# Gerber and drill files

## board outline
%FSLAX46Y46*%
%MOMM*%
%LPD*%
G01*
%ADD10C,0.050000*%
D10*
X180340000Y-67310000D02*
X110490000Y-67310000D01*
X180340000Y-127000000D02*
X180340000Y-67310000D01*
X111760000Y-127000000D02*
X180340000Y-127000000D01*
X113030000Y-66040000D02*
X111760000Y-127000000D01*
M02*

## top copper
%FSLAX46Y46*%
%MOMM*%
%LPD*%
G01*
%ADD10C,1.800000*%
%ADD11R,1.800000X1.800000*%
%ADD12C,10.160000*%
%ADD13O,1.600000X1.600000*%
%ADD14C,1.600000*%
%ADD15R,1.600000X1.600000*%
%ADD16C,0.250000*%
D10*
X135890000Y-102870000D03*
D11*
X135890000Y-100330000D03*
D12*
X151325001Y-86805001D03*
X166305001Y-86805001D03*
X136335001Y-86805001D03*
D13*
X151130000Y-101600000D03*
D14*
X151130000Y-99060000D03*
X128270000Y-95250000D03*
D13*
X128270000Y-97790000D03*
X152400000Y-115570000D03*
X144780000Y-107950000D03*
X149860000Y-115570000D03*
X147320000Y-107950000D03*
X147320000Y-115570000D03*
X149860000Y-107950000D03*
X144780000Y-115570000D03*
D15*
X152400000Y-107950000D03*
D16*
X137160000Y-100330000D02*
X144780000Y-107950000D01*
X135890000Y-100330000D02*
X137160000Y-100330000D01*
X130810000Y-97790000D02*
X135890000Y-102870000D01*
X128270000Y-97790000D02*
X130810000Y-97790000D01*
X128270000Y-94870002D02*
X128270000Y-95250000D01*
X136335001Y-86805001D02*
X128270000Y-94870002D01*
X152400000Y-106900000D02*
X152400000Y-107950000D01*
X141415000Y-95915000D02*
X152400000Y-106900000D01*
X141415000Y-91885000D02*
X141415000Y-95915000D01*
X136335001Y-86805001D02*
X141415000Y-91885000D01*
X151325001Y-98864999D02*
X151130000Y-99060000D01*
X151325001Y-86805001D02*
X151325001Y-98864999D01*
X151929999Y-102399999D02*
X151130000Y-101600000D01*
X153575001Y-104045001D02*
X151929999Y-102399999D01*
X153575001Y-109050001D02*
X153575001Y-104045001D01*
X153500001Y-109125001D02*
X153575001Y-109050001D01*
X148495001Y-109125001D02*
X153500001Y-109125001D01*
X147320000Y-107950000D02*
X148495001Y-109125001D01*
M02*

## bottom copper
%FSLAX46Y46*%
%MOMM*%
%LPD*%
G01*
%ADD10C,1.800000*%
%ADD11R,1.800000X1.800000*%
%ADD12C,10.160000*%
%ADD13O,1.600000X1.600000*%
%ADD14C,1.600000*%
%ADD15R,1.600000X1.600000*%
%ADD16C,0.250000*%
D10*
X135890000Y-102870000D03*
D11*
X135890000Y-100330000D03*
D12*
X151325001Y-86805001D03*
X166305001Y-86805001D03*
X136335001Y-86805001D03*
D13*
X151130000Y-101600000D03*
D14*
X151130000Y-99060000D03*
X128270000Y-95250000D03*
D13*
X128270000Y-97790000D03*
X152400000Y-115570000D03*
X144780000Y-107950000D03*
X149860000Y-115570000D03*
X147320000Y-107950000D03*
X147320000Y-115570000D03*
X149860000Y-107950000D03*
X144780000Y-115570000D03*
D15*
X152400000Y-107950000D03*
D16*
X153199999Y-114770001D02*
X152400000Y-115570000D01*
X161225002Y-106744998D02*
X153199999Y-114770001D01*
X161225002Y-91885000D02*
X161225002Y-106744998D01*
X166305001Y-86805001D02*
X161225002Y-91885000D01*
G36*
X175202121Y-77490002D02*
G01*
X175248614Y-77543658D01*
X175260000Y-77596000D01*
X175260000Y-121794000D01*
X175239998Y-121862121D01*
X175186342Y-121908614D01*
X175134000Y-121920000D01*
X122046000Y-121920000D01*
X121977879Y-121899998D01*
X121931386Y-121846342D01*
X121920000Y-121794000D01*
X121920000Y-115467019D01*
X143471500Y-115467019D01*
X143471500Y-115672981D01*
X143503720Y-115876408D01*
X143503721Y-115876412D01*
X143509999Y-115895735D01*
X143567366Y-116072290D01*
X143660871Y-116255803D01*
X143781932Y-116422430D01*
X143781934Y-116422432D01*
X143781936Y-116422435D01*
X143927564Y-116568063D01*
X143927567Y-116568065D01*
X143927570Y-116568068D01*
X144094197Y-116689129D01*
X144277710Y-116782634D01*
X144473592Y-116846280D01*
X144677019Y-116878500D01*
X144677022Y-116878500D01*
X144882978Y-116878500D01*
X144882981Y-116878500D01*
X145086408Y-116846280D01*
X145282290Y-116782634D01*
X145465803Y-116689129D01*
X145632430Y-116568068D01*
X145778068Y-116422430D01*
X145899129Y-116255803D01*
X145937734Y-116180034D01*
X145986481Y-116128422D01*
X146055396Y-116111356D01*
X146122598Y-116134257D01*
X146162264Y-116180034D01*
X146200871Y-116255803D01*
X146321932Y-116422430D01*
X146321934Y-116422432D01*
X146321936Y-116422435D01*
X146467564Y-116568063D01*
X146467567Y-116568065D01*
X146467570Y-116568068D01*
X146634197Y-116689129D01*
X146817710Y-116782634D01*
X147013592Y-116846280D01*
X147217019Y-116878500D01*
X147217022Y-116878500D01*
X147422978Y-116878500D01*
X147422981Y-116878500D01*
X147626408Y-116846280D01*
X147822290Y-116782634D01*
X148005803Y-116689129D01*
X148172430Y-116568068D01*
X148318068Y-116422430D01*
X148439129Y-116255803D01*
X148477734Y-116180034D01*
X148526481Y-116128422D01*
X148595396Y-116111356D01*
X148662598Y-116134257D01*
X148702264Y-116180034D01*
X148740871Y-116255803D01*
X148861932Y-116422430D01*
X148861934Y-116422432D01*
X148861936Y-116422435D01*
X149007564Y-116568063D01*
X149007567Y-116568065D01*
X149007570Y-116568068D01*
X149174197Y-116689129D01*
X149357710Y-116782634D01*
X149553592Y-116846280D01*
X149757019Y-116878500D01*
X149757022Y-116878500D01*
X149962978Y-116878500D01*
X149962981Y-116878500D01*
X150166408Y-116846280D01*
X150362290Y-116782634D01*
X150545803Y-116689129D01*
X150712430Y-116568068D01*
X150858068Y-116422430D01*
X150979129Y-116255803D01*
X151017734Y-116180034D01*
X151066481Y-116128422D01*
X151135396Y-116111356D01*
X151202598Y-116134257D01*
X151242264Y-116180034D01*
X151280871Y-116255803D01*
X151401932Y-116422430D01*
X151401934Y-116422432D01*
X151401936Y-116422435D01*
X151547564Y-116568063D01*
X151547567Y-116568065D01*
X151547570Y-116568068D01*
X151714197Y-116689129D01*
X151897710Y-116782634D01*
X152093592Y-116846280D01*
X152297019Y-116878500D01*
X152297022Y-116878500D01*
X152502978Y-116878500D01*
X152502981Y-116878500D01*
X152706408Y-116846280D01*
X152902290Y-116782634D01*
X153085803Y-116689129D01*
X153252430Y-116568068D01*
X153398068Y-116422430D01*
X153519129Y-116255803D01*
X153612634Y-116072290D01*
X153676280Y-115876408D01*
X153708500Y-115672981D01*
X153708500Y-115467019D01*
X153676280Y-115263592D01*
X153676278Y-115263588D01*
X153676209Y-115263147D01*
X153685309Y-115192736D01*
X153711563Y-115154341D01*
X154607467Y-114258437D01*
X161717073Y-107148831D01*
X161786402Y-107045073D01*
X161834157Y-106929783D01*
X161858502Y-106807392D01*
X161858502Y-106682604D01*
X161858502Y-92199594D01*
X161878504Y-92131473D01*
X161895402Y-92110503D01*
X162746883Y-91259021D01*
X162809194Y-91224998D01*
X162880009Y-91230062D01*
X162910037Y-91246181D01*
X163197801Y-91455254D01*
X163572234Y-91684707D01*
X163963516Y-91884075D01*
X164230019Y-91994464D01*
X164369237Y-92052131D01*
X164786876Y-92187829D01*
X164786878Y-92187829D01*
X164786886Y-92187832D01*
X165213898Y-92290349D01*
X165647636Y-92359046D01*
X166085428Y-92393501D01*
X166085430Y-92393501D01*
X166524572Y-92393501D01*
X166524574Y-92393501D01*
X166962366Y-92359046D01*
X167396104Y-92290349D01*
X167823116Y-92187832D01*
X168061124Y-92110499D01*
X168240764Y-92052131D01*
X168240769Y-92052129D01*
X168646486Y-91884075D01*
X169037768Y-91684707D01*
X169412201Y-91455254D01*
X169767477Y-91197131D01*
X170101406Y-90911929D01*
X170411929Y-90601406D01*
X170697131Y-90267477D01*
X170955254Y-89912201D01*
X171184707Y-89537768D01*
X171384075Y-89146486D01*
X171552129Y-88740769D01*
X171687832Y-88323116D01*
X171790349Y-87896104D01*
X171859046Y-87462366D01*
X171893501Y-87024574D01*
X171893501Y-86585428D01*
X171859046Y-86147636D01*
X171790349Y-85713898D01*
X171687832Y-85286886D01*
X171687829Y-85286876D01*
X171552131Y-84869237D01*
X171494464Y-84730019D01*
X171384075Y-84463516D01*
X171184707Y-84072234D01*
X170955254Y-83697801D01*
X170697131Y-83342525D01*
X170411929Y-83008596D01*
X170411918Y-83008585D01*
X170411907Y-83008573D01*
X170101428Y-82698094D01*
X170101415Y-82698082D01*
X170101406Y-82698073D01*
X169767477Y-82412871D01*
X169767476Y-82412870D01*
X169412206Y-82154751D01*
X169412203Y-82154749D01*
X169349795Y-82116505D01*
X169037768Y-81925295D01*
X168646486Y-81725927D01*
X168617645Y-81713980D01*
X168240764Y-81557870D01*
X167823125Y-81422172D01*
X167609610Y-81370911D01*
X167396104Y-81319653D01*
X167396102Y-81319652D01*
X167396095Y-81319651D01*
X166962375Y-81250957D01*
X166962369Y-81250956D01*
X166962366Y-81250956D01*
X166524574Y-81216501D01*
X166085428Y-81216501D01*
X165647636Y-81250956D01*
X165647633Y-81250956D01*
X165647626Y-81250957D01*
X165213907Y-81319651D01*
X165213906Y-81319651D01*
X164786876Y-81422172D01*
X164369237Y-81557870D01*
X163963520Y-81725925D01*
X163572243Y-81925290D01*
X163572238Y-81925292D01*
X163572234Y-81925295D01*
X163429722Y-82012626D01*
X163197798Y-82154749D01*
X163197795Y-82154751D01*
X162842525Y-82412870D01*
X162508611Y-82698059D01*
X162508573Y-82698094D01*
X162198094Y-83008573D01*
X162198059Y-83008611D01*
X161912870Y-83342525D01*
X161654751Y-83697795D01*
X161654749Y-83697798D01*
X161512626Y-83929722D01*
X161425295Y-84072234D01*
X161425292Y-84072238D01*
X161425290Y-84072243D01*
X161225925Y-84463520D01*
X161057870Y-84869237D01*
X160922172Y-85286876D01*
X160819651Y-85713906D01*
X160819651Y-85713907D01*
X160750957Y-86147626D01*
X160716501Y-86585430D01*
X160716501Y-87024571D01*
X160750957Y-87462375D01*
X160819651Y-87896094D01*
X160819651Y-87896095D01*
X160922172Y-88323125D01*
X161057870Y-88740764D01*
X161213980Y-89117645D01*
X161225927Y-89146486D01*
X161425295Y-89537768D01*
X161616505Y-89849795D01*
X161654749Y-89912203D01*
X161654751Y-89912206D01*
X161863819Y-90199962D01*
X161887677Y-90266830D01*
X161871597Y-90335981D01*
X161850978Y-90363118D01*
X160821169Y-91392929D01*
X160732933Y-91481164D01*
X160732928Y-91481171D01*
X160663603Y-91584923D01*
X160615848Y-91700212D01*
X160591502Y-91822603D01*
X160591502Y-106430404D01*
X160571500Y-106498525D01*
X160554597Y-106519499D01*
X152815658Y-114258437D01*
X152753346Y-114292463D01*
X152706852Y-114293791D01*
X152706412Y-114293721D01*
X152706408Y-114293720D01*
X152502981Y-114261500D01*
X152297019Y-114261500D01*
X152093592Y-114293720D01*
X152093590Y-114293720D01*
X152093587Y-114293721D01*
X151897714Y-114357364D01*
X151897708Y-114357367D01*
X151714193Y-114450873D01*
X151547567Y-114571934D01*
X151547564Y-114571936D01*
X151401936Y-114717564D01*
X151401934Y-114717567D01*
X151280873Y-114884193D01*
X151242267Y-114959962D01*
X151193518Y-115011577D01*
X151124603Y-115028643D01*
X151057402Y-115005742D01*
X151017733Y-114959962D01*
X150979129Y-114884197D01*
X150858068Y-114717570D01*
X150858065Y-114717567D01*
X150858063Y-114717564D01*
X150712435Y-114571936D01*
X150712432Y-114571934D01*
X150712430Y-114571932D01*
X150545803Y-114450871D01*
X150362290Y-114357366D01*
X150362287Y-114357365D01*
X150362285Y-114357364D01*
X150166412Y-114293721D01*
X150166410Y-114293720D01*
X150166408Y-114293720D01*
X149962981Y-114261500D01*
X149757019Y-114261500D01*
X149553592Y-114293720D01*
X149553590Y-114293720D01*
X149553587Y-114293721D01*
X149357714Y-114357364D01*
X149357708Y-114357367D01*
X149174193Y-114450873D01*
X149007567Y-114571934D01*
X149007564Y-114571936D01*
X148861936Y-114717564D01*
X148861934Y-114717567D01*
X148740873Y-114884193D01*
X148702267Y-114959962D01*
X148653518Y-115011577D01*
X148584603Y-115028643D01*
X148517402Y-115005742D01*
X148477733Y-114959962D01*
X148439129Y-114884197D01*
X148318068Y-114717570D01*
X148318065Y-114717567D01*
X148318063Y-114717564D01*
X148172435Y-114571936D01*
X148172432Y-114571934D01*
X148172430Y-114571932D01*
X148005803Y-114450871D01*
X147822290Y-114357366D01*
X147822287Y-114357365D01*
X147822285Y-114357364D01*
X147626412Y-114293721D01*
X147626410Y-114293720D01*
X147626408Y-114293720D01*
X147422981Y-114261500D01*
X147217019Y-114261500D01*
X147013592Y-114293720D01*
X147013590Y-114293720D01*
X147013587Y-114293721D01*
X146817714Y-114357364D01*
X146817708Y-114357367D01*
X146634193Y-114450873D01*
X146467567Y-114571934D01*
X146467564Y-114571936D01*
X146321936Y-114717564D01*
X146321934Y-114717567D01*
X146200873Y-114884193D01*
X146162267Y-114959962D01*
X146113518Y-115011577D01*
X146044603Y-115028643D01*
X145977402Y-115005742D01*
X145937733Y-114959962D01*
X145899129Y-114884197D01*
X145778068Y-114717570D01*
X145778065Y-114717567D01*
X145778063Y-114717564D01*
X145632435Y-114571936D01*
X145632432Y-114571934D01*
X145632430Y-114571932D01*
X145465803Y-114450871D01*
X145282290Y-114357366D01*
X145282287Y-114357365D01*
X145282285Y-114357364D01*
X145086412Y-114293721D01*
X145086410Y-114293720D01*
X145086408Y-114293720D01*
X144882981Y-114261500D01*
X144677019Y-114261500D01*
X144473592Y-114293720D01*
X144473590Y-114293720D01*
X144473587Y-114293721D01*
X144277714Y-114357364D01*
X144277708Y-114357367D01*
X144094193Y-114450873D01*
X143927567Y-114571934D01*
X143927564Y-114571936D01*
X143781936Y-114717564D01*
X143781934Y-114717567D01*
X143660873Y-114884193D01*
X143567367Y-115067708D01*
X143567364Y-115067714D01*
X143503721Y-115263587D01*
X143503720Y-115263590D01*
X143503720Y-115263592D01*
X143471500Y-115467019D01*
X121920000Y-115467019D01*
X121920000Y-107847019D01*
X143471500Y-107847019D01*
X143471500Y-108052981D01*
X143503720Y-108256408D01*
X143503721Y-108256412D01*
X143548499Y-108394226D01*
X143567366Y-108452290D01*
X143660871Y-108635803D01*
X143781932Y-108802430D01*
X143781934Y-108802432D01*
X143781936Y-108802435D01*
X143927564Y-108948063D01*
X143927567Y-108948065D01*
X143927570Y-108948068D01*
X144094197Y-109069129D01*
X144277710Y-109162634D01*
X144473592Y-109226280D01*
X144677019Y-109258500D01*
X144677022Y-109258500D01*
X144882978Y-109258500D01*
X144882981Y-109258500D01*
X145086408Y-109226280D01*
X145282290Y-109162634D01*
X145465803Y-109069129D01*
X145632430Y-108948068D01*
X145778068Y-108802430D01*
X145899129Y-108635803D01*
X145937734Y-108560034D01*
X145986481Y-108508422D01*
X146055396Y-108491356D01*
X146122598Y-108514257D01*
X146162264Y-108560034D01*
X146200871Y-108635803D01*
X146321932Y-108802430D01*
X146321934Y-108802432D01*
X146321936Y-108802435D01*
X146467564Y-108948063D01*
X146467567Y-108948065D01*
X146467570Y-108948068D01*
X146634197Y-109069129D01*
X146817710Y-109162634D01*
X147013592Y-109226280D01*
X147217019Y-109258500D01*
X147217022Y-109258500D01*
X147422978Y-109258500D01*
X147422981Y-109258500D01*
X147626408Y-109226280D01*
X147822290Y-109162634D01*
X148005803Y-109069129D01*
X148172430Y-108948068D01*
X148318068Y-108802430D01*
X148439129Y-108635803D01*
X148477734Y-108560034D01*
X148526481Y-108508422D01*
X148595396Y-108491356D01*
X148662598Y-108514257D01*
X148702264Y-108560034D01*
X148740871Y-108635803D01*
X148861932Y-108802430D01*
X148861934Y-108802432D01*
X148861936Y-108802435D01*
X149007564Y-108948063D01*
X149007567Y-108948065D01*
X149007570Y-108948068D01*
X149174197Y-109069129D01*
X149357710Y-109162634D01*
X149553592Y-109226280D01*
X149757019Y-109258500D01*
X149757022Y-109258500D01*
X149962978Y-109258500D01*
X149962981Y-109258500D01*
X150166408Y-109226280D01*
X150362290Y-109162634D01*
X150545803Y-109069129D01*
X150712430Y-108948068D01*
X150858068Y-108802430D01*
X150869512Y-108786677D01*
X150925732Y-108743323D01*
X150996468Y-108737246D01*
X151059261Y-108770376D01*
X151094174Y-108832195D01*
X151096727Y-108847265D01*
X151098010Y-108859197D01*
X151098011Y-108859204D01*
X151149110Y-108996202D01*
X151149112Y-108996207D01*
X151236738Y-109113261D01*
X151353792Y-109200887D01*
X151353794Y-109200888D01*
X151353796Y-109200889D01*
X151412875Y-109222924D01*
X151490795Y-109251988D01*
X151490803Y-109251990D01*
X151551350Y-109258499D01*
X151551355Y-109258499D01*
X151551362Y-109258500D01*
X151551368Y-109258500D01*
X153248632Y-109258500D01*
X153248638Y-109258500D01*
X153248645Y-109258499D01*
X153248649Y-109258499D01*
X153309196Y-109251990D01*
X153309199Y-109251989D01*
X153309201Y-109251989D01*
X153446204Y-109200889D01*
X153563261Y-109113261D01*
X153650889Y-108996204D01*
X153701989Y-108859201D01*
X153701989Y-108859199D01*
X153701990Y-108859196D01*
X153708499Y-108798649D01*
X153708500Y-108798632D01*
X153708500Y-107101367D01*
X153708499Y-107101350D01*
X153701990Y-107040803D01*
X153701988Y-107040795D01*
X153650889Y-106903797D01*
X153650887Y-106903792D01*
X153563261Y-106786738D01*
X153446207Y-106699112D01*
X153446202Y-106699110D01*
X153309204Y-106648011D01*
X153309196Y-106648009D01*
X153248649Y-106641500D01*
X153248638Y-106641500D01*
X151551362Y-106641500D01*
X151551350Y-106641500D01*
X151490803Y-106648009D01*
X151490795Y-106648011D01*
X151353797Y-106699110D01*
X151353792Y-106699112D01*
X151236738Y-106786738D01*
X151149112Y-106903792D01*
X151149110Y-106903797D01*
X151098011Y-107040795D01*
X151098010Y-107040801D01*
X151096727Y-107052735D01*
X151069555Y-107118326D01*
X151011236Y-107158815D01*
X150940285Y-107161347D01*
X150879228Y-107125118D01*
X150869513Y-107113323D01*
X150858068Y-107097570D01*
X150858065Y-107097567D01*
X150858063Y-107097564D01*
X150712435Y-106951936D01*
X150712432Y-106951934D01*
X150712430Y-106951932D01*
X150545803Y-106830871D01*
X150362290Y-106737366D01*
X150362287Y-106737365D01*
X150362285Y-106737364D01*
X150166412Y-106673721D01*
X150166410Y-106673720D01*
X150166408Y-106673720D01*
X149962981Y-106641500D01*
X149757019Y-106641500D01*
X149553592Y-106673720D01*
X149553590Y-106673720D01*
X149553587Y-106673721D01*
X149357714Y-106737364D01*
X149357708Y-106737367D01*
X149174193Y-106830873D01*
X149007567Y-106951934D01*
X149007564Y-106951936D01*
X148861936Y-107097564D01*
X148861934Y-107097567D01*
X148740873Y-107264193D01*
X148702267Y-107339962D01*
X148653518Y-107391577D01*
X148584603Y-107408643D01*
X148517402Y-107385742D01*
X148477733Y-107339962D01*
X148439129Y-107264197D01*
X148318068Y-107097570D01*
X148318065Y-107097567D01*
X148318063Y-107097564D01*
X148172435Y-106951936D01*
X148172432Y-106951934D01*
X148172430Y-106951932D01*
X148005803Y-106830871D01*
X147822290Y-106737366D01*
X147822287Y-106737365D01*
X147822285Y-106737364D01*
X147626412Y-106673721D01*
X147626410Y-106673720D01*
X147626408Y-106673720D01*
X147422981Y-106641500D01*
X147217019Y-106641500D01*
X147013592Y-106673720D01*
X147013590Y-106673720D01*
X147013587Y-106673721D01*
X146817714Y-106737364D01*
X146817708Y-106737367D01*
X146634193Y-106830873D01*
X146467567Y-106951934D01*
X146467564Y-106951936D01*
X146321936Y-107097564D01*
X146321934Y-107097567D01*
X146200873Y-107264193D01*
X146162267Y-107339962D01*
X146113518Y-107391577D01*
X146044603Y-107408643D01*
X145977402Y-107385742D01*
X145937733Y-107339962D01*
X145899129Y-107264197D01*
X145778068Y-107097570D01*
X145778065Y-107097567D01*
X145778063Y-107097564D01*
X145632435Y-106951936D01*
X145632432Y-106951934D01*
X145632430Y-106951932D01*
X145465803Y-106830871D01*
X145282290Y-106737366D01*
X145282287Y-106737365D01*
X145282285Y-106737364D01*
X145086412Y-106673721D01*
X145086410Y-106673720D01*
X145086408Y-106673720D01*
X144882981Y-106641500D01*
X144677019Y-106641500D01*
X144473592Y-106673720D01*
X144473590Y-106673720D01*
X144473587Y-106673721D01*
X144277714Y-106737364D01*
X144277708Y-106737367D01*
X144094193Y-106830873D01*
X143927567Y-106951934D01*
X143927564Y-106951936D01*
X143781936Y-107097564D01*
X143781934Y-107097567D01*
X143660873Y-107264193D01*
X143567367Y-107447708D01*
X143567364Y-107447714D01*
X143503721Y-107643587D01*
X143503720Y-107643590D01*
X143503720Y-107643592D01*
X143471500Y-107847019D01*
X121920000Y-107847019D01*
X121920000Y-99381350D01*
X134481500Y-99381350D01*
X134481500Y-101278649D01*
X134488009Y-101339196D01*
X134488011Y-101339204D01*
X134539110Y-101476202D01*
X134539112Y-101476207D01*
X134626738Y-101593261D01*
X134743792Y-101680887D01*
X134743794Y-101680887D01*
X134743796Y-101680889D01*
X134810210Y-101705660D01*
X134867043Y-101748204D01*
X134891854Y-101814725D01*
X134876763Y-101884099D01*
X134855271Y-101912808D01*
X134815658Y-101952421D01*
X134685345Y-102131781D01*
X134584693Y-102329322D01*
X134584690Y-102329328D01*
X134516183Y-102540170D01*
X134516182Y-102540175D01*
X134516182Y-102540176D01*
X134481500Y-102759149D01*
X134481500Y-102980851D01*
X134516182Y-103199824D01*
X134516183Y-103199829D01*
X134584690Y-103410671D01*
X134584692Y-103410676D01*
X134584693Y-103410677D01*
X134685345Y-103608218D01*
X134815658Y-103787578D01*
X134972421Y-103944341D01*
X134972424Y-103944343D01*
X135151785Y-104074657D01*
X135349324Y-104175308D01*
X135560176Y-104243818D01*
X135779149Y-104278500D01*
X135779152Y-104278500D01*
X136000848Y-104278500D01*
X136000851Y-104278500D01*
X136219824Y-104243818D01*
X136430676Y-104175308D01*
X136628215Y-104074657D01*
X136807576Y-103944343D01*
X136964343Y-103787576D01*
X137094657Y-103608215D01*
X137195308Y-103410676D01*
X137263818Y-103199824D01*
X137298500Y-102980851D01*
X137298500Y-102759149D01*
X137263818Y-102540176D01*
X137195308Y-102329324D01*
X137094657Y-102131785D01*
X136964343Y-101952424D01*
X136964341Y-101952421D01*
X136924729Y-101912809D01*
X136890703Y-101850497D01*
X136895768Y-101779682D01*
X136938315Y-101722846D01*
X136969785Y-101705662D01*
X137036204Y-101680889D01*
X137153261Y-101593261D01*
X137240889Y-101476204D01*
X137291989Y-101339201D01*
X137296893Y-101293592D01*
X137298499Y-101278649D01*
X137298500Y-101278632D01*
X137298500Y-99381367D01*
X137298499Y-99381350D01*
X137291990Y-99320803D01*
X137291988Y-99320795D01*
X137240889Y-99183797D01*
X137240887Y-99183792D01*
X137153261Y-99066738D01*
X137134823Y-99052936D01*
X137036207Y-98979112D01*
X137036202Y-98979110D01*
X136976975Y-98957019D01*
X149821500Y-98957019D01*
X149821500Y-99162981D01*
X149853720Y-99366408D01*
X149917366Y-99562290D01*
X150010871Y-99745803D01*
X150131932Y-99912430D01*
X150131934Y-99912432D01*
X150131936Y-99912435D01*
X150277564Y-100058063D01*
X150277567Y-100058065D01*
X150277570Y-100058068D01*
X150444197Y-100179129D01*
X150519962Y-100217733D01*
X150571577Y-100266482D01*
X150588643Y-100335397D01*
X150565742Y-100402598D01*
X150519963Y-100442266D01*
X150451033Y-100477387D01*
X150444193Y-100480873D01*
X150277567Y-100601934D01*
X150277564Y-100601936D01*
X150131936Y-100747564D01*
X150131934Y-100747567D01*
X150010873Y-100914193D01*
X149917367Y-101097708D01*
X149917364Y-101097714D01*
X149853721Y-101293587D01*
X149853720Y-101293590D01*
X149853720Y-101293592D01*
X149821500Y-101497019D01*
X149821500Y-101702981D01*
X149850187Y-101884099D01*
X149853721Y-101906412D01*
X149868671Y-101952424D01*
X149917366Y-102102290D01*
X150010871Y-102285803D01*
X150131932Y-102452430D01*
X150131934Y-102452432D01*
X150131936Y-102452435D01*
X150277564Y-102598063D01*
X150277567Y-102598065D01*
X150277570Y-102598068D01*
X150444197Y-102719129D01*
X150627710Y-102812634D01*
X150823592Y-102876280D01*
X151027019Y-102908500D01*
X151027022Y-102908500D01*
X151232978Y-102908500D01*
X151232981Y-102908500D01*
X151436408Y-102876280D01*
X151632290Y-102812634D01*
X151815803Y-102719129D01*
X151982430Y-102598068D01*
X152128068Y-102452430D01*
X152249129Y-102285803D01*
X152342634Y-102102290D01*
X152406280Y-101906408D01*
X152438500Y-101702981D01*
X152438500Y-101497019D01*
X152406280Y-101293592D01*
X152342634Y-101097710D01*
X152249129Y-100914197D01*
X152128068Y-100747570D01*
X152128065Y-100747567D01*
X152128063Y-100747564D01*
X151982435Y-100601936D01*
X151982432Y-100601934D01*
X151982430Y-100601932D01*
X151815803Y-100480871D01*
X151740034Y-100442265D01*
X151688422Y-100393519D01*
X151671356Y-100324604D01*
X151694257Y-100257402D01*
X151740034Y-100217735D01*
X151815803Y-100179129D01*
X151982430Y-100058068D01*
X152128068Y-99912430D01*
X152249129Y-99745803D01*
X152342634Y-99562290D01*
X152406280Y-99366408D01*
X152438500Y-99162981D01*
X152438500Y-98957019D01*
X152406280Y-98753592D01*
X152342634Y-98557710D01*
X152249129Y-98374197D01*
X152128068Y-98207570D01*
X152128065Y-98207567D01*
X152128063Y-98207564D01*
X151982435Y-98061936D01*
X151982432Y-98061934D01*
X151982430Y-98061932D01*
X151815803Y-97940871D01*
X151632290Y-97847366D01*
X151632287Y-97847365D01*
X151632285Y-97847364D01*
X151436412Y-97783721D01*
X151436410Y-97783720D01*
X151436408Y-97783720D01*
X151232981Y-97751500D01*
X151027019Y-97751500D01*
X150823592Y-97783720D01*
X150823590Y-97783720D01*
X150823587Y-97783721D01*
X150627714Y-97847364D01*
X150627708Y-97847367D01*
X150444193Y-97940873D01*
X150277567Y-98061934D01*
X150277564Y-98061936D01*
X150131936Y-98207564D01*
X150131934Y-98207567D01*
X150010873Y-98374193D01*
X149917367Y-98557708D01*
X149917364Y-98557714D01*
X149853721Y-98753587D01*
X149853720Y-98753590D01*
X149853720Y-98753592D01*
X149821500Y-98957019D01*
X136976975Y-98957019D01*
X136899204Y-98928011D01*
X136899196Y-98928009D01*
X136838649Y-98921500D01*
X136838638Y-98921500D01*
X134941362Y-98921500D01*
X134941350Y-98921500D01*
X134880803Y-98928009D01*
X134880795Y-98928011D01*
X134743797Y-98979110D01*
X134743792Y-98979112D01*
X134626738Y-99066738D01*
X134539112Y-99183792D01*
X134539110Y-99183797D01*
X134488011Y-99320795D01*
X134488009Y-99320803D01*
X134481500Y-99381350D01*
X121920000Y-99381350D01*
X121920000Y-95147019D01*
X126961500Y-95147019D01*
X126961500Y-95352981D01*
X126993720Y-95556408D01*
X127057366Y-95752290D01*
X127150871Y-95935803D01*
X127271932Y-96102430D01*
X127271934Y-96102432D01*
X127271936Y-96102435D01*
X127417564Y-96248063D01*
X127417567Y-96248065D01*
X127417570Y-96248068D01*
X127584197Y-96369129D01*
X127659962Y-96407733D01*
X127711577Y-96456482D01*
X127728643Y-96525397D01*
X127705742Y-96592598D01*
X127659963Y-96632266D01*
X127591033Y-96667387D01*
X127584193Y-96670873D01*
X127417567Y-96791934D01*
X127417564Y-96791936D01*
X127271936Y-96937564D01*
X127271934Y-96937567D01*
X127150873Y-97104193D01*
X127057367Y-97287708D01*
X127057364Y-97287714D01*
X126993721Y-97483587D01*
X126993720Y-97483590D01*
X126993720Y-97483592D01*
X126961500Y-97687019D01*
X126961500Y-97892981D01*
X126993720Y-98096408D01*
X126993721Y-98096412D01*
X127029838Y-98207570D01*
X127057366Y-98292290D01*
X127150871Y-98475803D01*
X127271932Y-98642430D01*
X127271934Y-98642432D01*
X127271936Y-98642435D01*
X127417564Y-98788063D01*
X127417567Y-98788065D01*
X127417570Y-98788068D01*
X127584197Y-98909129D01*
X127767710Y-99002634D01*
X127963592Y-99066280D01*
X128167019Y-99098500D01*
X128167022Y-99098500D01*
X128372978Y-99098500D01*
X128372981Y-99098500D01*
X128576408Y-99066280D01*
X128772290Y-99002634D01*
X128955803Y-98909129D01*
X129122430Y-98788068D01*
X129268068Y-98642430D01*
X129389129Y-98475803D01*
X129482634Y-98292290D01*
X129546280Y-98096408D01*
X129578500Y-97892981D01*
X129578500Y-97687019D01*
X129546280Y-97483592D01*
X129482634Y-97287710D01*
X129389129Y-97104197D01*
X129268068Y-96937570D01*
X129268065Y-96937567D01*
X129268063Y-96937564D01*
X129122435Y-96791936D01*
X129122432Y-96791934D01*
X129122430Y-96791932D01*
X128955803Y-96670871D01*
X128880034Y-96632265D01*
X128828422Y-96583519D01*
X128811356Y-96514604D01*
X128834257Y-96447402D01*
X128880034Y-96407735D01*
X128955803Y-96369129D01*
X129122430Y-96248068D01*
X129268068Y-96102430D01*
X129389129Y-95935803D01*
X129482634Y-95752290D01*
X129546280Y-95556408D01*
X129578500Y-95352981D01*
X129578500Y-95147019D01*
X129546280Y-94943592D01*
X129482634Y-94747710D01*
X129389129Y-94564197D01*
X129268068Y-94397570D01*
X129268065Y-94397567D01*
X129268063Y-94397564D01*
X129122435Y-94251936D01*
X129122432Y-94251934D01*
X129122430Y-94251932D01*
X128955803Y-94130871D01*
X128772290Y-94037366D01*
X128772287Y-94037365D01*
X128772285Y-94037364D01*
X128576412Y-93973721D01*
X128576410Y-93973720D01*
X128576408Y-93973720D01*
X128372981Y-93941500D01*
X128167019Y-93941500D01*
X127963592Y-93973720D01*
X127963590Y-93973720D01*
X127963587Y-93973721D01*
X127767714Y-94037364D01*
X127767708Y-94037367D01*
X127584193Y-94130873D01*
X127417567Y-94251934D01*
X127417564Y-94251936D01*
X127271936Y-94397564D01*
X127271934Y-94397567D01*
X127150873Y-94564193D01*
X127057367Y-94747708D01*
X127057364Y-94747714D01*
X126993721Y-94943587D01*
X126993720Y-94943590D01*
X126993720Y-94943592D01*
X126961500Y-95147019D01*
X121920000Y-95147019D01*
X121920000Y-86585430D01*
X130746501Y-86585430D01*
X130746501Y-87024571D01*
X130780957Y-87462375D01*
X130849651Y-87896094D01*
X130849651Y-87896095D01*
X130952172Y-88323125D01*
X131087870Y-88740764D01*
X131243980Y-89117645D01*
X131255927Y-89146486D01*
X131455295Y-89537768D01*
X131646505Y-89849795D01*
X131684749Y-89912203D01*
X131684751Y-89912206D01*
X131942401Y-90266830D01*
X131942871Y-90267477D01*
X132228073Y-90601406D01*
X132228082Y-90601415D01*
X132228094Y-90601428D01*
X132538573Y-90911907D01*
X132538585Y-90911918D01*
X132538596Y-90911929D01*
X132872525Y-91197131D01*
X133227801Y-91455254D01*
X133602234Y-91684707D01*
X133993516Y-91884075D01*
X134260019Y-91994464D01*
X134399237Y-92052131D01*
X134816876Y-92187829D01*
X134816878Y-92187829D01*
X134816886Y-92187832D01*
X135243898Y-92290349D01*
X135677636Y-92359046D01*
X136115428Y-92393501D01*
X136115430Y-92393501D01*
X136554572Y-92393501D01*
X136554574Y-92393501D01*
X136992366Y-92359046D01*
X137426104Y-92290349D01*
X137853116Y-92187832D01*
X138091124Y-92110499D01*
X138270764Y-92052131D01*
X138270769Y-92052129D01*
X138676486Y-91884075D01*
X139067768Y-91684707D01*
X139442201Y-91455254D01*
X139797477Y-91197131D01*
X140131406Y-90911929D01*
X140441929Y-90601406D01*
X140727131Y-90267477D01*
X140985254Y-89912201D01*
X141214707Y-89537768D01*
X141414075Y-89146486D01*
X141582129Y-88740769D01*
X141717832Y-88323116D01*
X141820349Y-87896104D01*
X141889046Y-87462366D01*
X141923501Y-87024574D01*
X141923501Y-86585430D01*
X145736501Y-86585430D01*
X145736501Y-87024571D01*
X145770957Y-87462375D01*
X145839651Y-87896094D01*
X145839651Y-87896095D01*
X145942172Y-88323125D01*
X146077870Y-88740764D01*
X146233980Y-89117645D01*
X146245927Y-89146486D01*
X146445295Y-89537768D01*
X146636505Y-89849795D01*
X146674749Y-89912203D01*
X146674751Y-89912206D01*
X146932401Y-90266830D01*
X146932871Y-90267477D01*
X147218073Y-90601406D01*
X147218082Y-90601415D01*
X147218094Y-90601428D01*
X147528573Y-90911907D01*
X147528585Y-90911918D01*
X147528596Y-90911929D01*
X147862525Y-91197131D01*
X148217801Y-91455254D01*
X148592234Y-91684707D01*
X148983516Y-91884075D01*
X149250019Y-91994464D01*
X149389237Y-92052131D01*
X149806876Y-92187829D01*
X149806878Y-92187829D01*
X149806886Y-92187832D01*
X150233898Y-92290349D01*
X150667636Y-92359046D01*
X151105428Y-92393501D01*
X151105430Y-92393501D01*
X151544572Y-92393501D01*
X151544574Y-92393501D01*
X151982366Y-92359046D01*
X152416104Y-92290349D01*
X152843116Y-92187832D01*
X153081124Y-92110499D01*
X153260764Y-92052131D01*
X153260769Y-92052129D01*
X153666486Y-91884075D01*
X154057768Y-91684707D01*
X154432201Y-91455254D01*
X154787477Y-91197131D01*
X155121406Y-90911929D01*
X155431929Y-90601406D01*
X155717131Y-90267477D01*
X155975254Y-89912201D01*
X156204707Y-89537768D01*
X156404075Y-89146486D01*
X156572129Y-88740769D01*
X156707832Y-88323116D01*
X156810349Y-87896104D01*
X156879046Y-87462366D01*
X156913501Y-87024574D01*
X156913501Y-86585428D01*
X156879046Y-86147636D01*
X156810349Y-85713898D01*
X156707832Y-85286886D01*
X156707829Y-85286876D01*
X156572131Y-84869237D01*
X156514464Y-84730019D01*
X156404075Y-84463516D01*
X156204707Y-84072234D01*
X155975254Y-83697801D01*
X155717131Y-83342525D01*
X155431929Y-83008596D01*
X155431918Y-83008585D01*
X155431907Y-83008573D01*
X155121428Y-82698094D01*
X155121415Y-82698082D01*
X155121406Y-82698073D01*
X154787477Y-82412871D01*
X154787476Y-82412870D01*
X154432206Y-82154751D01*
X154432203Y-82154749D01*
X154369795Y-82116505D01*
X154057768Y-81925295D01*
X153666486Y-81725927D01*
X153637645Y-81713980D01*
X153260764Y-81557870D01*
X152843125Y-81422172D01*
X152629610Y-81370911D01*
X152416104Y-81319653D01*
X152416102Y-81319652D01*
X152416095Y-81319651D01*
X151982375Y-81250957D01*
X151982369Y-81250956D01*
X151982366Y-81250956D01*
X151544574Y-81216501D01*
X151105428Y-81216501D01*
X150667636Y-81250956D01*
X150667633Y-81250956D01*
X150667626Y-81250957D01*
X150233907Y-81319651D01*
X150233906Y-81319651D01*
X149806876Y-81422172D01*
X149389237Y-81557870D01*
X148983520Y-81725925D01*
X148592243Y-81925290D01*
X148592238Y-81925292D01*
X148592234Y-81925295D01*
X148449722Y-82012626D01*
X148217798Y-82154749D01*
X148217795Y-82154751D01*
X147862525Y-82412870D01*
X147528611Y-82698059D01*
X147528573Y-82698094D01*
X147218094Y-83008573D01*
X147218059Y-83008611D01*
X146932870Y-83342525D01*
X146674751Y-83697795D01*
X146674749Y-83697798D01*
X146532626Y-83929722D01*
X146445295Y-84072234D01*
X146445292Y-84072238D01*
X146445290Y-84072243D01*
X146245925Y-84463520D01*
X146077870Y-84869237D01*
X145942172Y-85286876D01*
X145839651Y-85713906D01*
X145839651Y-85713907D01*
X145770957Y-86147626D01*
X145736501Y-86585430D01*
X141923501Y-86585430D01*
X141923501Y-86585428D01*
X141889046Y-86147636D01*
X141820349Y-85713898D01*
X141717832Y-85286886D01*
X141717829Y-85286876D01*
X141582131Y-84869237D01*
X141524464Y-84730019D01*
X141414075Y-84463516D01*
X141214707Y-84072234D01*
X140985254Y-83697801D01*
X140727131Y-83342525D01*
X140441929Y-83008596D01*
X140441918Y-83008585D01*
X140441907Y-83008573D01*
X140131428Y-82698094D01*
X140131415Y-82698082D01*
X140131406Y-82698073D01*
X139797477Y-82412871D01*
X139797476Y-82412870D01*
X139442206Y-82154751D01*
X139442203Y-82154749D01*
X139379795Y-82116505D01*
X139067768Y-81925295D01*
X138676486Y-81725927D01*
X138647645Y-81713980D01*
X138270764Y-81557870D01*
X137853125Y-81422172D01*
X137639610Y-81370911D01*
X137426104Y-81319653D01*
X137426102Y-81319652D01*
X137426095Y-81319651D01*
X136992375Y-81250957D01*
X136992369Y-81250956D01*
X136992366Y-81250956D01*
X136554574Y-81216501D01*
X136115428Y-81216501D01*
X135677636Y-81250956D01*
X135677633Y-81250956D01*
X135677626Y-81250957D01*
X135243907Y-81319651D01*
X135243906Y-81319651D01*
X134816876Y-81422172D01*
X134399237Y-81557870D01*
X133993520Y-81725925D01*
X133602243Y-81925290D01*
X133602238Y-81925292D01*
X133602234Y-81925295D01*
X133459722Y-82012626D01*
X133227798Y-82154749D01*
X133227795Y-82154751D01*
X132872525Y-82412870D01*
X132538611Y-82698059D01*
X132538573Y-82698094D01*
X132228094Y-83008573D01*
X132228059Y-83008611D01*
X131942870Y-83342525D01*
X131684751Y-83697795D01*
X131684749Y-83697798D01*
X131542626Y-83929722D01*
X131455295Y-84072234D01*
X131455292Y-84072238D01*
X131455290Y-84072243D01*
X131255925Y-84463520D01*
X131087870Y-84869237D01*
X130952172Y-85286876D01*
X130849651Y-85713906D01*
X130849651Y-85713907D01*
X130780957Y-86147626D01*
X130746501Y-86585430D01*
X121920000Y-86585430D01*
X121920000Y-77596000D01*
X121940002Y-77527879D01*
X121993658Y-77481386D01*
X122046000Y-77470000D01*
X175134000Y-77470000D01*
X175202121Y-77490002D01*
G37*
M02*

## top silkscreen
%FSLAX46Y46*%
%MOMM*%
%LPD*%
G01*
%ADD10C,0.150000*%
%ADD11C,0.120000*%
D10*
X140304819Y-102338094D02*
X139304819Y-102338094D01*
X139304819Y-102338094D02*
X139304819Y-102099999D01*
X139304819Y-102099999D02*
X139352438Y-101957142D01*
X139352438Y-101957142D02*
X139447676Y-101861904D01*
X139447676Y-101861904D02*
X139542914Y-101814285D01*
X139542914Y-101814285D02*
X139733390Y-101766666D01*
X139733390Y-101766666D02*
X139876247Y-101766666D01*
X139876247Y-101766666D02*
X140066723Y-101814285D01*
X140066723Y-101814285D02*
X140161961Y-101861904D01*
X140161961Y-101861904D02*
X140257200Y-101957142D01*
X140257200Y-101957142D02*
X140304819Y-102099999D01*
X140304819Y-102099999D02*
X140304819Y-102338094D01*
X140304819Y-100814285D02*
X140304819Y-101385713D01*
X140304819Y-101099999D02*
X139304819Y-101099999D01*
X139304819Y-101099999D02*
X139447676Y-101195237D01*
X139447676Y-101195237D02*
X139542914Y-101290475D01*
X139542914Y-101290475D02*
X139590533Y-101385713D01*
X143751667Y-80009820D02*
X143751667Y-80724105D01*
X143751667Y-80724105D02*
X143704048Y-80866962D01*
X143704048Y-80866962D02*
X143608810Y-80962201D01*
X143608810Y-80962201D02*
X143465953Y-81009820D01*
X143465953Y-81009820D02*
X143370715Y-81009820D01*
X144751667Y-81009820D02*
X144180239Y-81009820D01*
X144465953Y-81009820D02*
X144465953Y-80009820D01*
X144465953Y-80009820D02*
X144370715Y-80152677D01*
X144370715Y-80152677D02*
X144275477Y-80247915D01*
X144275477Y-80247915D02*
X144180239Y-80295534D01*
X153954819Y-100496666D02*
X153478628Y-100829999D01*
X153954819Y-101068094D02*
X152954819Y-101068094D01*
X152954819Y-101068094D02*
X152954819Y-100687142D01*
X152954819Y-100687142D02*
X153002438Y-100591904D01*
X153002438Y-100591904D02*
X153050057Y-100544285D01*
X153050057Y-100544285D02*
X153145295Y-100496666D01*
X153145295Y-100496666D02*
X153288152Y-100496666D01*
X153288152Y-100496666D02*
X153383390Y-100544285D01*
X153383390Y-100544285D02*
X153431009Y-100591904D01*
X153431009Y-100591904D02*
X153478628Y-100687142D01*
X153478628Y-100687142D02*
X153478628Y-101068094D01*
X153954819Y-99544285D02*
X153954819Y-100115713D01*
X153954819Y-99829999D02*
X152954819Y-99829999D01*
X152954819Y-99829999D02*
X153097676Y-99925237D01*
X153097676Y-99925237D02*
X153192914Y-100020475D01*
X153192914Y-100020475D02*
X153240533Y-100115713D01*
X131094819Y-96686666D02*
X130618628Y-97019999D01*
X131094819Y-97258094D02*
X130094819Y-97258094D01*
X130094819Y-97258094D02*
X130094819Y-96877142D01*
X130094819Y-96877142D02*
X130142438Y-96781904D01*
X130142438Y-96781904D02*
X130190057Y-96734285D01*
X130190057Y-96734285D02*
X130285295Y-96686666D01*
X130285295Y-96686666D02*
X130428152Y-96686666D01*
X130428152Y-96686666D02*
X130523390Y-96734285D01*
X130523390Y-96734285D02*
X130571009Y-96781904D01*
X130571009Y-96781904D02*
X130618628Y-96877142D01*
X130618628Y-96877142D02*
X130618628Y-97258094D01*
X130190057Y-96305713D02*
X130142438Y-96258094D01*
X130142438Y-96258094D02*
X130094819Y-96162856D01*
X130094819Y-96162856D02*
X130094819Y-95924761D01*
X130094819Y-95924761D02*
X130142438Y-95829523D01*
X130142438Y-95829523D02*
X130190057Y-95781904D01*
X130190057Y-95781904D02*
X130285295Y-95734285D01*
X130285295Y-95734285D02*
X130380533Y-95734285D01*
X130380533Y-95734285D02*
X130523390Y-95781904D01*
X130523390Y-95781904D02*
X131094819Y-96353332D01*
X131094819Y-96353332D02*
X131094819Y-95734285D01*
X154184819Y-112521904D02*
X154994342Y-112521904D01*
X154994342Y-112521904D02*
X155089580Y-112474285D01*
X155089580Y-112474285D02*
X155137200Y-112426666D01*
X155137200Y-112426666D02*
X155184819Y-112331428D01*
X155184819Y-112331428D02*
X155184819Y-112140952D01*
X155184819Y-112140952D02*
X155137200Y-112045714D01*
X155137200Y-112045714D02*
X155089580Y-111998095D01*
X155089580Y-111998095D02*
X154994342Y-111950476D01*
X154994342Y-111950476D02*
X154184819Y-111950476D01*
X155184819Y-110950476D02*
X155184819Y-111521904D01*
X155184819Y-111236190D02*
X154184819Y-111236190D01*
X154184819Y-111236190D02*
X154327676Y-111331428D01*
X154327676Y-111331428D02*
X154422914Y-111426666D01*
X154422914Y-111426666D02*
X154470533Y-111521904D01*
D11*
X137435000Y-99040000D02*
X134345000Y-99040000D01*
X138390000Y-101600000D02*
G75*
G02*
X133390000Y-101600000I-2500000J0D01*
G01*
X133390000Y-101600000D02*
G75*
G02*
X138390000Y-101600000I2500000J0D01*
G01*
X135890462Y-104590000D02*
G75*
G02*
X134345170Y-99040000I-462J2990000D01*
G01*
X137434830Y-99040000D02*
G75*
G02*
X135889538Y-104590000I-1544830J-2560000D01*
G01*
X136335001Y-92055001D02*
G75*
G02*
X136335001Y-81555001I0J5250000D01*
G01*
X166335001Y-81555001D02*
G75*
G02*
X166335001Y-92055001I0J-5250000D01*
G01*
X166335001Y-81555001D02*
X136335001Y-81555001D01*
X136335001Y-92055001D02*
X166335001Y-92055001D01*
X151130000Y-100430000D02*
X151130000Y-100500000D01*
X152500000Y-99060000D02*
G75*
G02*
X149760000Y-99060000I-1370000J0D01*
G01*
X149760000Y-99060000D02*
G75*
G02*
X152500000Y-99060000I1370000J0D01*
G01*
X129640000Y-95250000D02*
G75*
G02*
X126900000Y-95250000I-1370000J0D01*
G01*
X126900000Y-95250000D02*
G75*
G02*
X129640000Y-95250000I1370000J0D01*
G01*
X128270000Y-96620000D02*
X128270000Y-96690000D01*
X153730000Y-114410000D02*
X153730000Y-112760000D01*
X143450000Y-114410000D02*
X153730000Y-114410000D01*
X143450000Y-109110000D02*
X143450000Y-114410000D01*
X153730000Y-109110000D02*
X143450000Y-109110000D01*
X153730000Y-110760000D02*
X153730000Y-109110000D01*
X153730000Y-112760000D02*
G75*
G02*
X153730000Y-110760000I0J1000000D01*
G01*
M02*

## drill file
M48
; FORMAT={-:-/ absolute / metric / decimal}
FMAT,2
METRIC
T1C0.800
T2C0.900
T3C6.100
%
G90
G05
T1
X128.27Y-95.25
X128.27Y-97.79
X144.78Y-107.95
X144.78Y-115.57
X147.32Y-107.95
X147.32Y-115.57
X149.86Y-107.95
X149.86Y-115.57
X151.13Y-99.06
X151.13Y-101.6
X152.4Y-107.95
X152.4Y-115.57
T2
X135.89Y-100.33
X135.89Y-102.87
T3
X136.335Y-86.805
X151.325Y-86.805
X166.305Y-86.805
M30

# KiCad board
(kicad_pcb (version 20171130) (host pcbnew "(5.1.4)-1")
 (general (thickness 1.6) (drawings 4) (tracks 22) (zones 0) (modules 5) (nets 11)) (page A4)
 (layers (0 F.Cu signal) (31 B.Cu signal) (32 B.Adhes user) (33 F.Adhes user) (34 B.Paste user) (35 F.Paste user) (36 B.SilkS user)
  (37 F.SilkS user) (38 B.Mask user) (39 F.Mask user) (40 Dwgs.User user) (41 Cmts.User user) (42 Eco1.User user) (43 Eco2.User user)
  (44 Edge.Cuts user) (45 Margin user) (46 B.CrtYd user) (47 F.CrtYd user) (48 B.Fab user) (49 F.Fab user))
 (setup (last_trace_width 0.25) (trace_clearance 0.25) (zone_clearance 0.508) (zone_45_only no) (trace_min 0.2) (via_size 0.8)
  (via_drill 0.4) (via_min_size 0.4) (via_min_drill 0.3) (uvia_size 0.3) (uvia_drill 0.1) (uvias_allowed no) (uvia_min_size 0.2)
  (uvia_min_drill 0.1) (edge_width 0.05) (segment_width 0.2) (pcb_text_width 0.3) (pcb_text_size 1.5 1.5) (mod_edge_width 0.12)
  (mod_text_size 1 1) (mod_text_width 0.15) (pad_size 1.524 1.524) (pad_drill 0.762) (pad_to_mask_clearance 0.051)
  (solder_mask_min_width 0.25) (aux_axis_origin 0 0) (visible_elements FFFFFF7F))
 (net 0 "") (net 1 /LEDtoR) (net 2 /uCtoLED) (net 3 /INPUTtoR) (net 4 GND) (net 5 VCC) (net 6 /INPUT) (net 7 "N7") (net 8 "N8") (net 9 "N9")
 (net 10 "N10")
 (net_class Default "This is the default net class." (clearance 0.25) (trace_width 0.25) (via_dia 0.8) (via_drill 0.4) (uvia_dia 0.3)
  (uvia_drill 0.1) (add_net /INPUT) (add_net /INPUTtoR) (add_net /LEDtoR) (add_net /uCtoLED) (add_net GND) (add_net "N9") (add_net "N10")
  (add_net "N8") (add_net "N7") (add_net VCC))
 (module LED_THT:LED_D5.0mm (layer F.Cu) (at 135.89 100.33 270)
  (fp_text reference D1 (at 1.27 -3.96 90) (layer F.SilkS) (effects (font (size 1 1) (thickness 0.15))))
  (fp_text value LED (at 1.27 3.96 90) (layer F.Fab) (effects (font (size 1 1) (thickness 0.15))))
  (fp_line (start -1.29 -1.545) (end -1.29 1.545) (layer F.SilkS) (width 0.12))
  (fp_circle (center 1.27 0) (end 3.77 0) (layer F.SilkS) (width 0.12))
  (fp_arc (start 1.27 0) (end -1.29 1.54483) (angle -148.9) (layer F.SilkS) (width 0.12))
  (fp_arc (start 1.27 0) (end -1.29 -1.54483) (angle 148.9) (layer F.SilkS) (width 0.12))
  (pad 2 thru_hole circle (at 2.54 0 270) (size 1.8 1.8) (drill 0.9) (layers *.Cu *.Mask) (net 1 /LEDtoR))
  (pad 1 thru_hole rect (at 0 0 270) (size 1.8 1.8) (drill 0.9) (layers *.Cu *.Mask) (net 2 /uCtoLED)))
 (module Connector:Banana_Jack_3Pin (layer F.Cu) (at 136.335001 86.805001)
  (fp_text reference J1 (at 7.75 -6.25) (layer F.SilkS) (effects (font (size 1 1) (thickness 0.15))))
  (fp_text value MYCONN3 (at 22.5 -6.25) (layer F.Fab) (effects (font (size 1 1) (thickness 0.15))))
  (fp_arc (start 0 0) (end 0 5.25) (angle 180) (layer F.SilkS) (width 0.12))
  (fp_arc (start 30 0) (end 30 -5.25) (angle 180) (layer F.SilkS) (width 0.12))
  (fp_line (start 30 -5.25) (end 0 -5.25) (layer F.SilkS) (width 0.12))
  (fp_line (start 0 5.25) (end 30 5.25) (layer F.SilkS) (width 0.12))
  (pad 2 thru_hole circle (at 14.99 0) (size 10.16 10.16) (drill 6.1) (layers *.Cu *.Mask) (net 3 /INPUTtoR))
  (pad 3 thru_hole circle (at 29.97 0) (size 10.16 10.16) (drill 6.1) (layers *.Cu *.Mask) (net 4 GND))
  (pad 1 thru_hole circle (at 0 0) (size 10.16 10.16) (drill 6.1) (layers *.Cu *.Mask) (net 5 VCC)))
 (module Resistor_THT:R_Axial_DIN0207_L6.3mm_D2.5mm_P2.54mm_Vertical (layer F.Cu) (at 151.13 99.06 270)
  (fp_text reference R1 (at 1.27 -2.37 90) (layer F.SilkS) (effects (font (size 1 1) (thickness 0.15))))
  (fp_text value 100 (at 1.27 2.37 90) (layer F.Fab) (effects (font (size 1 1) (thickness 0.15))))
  (fp_line (start 1.37 0) (end 1.44 0) (layer F.SilkS) (width 0.12))
  (fp_circle (center 0 0) (end 1.37 0) (layer F.SilkS) (width 0.12))
  (pad 2 thru_hole oval (at 2.54 0 270) (size 1.6 1.6) (drill 0.8) (layers *.Cu *.Mask) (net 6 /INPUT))
  (pad 1 thru_hole circle (at 0 0 270) (size 1.6 1.6) (drill 0.8) (layers *.Cu *.Mask) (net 3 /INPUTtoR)))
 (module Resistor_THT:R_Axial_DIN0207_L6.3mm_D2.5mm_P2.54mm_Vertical (layer F.Cu) (at 128.27 95.25 270)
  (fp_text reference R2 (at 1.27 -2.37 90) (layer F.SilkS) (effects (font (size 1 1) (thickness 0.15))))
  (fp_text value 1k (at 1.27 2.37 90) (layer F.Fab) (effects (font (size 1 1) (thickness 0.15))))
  (fp_circle (center 0 0) (end 1.37 0) (layer F.SilkS) (width 0.12))
  (fp_line (start 1.37 0) (end 1.44 0) (layer F.SilkS) (width 0.12))
  (pad 1 thru_hole circle (at 0 0 270) (size 1.6 1.6) (drill 0.8) (layers *.Cu *.Mask) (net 5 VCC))
  (pad 2 thru_hole oval (at 2.54 0 270) (size 1.6 1.6) (drill 0.8) (layers *.Cu *.Mask) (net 1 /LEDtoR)))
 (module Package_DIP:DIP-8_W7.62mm (layer F.Cu) (at 152.4 107.95 270)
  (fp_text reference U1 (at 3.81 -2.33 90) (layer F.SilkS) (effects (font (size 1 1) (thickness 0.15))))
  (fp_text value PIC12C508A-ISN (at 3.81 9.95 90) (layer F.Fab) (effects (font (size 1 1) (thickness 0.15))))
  (fp_line (start 6.46 -1.33) (end 4.81 -1.33) (layer F.SilkS) (width 0.12))
  (fp_line (start 6.46 8.95) (end 6.46 -1.33) (layer F.SilkS) (width 0.12))
  (fp_line (start 1.16 8.95) (end 6.46 8.95) (layer F.SilkS) (width 0.12))
  (fp_line (start 1.16 -1.33) (end 1.16 8.95) (layer F.SilkS) (width 0.12))
  (fp_line (start 2.81 -1.33) (end 1.16 -1.33) (layer F.SilkS) (width 0.12))
  (fp_arc (start 3.81 -1.33) (end 2.81 -1.33) (angle -180) (layer F.SilkS) (width 0.12))
  (pad 8 thru_hole oval (at 7.62 0 270) (size 1.6 1.6) (drill 0.8) (layers *.Cu *.Mask) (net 4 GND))
  (pad 4 thru_hole oval (at 0 7.62 270) (size 1.6 1.6) (drill 0.8) (layers *.Cu *.Mask) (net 2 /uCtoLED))
  (pad 7 thru_hole oval (at 7.62 2.54 270) (size 1.6 1.6) (drill 0.8) (layers *.Cu *.Mask) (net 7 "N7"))
  (pad 3 thru_hole oval (at 0 5.08 270) (size 1.6 1.6) (drill 0.8) (layers *.Cu *.Mask) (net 6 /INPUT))
  (pad 6 thru_hole oval (at 7.62 5.08 270) (size 1.6 1.6) (drill 0.8) (layers *.Cu *.Mask) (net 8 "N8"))
  (pad 2 thru_hole oval (at 0 2.54 270) (size 1.6 1.6) (drill 0.8) (layers *.Cu *.Mask) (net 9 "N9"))
  (pad 5 thru_hole oval (at 7.62 7.62 270) (size 1.6 1.6) (drill 0.8) (layers *.Cu *.Mask) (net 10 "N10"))
  (pad 1 thru_hole rect (at 0 0 270) (size 1.6 1.6) (drill 0.8) (layers *.Cu *.Mask) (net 5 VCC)))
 (gr_line (start 180.34 67.31) (end 110.49 67.31) (layer Edge.Cuts) (width 0.05))
 (gr_line (start 180.34 127) (end 180.34 67.31) (layer Edge.Cuts) (width 0.05))
 (gr_line (start 111.76 127) (end 180.34 127) (layer Edge.Cuts) (width 0.05))
 (gr_line (start 113.03 66.04) (end 111.76 127) (layer Edge.Cuts) (width 0.05))
 (segment (start 137.16 100.33) (end 144.78 107.95) (width 0.25) (layer F.Cu) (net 2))
 (segment (start 135.89 100.33) (end 137.16 100.33) (width 0.25) (layer F.Cu) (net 2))
 (segment (start 130.81 97.79) (end 135.89 102.87) (width 0.25) (layer F.Cu) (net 1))
 (segment (start 128.27 97.79) (end 130.81 97.79) (width 0.25) (layer F.Cu) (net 1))
 (segment (start 128.27 94.870002) (end 128.27 95.25) (width 0.25) (layer F.Cu) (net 5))
 (segment (start 136.335001 86.805001) (end 128.27 94.870002) (width 0.25) (layer F.Cu) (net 5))
 (segment (start 152.4 106.9) (end 152.4 107.95) (width 0.25) (layer F.Cu) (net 5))
 (segment (start 141.415 95.915) (end 152.4 106.9) (width 0.25) (layer F.Cu) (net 5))
 (segment (start 141.415 91.885) (end 141.415 95.915) (width 0.25) (layer F.Cu) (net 5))
 (segment (start 136.335001 86.805001) (end 141.415 91.885) (width 0.25) (layer F.Cu) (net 5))
 (segment (start 153.199999 114.770001) (end 152.4 115.57) (width 0.25) (layer B.Cu) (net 4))
 (segment (start 161.225002 106.744998) (end 153.199999 114.770001) (width 0.25) (layer B.Cu) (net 4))
 (segment (start 161.225002 91.885) (end 161.225002 106.744998) (width 0.25) (layer B.Cu) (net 4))
 (segment (start 166.305001 86.805001) (end 161.225002 91.885) (width 0.25) (layer B.Cu) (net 4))
 (segment (start 151.325001 98.864999) (end 151.13 99.06) (width 0.25) (layer F.Cu) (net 3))
 (segment (start 151.325001 86.805001) (end 151.325001 98.864999) (width 0.25) (layer F.Cu) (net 3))
 (segment (start 151.929999 102.399999) (end 151.13 101.6) (width 0.25) (layer F.Cu) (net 6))
 (segment (start 153.575001 104.045001) (end 151.929999 102.399999) (width 0.25) (layer F.Cu) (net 6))
 (segment (start 153.575001 109.050001) (end 153.575001 104.045001) (width 0.25) (layer F.Cu) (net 6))
 (segment (start 153.500001 109.125001) (end 153.575001 109.050001) (width 0.25) (layer F.Cu) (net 6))
 (segment (start 148.495001 109.125001) (end 153.500001 109.125001) (width 0.25) (layer F.Cu) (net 6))
 (segment (start 147.32 107.95) (end 148.495001 109.125001) (width 0.25) (layer F.Cu) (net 6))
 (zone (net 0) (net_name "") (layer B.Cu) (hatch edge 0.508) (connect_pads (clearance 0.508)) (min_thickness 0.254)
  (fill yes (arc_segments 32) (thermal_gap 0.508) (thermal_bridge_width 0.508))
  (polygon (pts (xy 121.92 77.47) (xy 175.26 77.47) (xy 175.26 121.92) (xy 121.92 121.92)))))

